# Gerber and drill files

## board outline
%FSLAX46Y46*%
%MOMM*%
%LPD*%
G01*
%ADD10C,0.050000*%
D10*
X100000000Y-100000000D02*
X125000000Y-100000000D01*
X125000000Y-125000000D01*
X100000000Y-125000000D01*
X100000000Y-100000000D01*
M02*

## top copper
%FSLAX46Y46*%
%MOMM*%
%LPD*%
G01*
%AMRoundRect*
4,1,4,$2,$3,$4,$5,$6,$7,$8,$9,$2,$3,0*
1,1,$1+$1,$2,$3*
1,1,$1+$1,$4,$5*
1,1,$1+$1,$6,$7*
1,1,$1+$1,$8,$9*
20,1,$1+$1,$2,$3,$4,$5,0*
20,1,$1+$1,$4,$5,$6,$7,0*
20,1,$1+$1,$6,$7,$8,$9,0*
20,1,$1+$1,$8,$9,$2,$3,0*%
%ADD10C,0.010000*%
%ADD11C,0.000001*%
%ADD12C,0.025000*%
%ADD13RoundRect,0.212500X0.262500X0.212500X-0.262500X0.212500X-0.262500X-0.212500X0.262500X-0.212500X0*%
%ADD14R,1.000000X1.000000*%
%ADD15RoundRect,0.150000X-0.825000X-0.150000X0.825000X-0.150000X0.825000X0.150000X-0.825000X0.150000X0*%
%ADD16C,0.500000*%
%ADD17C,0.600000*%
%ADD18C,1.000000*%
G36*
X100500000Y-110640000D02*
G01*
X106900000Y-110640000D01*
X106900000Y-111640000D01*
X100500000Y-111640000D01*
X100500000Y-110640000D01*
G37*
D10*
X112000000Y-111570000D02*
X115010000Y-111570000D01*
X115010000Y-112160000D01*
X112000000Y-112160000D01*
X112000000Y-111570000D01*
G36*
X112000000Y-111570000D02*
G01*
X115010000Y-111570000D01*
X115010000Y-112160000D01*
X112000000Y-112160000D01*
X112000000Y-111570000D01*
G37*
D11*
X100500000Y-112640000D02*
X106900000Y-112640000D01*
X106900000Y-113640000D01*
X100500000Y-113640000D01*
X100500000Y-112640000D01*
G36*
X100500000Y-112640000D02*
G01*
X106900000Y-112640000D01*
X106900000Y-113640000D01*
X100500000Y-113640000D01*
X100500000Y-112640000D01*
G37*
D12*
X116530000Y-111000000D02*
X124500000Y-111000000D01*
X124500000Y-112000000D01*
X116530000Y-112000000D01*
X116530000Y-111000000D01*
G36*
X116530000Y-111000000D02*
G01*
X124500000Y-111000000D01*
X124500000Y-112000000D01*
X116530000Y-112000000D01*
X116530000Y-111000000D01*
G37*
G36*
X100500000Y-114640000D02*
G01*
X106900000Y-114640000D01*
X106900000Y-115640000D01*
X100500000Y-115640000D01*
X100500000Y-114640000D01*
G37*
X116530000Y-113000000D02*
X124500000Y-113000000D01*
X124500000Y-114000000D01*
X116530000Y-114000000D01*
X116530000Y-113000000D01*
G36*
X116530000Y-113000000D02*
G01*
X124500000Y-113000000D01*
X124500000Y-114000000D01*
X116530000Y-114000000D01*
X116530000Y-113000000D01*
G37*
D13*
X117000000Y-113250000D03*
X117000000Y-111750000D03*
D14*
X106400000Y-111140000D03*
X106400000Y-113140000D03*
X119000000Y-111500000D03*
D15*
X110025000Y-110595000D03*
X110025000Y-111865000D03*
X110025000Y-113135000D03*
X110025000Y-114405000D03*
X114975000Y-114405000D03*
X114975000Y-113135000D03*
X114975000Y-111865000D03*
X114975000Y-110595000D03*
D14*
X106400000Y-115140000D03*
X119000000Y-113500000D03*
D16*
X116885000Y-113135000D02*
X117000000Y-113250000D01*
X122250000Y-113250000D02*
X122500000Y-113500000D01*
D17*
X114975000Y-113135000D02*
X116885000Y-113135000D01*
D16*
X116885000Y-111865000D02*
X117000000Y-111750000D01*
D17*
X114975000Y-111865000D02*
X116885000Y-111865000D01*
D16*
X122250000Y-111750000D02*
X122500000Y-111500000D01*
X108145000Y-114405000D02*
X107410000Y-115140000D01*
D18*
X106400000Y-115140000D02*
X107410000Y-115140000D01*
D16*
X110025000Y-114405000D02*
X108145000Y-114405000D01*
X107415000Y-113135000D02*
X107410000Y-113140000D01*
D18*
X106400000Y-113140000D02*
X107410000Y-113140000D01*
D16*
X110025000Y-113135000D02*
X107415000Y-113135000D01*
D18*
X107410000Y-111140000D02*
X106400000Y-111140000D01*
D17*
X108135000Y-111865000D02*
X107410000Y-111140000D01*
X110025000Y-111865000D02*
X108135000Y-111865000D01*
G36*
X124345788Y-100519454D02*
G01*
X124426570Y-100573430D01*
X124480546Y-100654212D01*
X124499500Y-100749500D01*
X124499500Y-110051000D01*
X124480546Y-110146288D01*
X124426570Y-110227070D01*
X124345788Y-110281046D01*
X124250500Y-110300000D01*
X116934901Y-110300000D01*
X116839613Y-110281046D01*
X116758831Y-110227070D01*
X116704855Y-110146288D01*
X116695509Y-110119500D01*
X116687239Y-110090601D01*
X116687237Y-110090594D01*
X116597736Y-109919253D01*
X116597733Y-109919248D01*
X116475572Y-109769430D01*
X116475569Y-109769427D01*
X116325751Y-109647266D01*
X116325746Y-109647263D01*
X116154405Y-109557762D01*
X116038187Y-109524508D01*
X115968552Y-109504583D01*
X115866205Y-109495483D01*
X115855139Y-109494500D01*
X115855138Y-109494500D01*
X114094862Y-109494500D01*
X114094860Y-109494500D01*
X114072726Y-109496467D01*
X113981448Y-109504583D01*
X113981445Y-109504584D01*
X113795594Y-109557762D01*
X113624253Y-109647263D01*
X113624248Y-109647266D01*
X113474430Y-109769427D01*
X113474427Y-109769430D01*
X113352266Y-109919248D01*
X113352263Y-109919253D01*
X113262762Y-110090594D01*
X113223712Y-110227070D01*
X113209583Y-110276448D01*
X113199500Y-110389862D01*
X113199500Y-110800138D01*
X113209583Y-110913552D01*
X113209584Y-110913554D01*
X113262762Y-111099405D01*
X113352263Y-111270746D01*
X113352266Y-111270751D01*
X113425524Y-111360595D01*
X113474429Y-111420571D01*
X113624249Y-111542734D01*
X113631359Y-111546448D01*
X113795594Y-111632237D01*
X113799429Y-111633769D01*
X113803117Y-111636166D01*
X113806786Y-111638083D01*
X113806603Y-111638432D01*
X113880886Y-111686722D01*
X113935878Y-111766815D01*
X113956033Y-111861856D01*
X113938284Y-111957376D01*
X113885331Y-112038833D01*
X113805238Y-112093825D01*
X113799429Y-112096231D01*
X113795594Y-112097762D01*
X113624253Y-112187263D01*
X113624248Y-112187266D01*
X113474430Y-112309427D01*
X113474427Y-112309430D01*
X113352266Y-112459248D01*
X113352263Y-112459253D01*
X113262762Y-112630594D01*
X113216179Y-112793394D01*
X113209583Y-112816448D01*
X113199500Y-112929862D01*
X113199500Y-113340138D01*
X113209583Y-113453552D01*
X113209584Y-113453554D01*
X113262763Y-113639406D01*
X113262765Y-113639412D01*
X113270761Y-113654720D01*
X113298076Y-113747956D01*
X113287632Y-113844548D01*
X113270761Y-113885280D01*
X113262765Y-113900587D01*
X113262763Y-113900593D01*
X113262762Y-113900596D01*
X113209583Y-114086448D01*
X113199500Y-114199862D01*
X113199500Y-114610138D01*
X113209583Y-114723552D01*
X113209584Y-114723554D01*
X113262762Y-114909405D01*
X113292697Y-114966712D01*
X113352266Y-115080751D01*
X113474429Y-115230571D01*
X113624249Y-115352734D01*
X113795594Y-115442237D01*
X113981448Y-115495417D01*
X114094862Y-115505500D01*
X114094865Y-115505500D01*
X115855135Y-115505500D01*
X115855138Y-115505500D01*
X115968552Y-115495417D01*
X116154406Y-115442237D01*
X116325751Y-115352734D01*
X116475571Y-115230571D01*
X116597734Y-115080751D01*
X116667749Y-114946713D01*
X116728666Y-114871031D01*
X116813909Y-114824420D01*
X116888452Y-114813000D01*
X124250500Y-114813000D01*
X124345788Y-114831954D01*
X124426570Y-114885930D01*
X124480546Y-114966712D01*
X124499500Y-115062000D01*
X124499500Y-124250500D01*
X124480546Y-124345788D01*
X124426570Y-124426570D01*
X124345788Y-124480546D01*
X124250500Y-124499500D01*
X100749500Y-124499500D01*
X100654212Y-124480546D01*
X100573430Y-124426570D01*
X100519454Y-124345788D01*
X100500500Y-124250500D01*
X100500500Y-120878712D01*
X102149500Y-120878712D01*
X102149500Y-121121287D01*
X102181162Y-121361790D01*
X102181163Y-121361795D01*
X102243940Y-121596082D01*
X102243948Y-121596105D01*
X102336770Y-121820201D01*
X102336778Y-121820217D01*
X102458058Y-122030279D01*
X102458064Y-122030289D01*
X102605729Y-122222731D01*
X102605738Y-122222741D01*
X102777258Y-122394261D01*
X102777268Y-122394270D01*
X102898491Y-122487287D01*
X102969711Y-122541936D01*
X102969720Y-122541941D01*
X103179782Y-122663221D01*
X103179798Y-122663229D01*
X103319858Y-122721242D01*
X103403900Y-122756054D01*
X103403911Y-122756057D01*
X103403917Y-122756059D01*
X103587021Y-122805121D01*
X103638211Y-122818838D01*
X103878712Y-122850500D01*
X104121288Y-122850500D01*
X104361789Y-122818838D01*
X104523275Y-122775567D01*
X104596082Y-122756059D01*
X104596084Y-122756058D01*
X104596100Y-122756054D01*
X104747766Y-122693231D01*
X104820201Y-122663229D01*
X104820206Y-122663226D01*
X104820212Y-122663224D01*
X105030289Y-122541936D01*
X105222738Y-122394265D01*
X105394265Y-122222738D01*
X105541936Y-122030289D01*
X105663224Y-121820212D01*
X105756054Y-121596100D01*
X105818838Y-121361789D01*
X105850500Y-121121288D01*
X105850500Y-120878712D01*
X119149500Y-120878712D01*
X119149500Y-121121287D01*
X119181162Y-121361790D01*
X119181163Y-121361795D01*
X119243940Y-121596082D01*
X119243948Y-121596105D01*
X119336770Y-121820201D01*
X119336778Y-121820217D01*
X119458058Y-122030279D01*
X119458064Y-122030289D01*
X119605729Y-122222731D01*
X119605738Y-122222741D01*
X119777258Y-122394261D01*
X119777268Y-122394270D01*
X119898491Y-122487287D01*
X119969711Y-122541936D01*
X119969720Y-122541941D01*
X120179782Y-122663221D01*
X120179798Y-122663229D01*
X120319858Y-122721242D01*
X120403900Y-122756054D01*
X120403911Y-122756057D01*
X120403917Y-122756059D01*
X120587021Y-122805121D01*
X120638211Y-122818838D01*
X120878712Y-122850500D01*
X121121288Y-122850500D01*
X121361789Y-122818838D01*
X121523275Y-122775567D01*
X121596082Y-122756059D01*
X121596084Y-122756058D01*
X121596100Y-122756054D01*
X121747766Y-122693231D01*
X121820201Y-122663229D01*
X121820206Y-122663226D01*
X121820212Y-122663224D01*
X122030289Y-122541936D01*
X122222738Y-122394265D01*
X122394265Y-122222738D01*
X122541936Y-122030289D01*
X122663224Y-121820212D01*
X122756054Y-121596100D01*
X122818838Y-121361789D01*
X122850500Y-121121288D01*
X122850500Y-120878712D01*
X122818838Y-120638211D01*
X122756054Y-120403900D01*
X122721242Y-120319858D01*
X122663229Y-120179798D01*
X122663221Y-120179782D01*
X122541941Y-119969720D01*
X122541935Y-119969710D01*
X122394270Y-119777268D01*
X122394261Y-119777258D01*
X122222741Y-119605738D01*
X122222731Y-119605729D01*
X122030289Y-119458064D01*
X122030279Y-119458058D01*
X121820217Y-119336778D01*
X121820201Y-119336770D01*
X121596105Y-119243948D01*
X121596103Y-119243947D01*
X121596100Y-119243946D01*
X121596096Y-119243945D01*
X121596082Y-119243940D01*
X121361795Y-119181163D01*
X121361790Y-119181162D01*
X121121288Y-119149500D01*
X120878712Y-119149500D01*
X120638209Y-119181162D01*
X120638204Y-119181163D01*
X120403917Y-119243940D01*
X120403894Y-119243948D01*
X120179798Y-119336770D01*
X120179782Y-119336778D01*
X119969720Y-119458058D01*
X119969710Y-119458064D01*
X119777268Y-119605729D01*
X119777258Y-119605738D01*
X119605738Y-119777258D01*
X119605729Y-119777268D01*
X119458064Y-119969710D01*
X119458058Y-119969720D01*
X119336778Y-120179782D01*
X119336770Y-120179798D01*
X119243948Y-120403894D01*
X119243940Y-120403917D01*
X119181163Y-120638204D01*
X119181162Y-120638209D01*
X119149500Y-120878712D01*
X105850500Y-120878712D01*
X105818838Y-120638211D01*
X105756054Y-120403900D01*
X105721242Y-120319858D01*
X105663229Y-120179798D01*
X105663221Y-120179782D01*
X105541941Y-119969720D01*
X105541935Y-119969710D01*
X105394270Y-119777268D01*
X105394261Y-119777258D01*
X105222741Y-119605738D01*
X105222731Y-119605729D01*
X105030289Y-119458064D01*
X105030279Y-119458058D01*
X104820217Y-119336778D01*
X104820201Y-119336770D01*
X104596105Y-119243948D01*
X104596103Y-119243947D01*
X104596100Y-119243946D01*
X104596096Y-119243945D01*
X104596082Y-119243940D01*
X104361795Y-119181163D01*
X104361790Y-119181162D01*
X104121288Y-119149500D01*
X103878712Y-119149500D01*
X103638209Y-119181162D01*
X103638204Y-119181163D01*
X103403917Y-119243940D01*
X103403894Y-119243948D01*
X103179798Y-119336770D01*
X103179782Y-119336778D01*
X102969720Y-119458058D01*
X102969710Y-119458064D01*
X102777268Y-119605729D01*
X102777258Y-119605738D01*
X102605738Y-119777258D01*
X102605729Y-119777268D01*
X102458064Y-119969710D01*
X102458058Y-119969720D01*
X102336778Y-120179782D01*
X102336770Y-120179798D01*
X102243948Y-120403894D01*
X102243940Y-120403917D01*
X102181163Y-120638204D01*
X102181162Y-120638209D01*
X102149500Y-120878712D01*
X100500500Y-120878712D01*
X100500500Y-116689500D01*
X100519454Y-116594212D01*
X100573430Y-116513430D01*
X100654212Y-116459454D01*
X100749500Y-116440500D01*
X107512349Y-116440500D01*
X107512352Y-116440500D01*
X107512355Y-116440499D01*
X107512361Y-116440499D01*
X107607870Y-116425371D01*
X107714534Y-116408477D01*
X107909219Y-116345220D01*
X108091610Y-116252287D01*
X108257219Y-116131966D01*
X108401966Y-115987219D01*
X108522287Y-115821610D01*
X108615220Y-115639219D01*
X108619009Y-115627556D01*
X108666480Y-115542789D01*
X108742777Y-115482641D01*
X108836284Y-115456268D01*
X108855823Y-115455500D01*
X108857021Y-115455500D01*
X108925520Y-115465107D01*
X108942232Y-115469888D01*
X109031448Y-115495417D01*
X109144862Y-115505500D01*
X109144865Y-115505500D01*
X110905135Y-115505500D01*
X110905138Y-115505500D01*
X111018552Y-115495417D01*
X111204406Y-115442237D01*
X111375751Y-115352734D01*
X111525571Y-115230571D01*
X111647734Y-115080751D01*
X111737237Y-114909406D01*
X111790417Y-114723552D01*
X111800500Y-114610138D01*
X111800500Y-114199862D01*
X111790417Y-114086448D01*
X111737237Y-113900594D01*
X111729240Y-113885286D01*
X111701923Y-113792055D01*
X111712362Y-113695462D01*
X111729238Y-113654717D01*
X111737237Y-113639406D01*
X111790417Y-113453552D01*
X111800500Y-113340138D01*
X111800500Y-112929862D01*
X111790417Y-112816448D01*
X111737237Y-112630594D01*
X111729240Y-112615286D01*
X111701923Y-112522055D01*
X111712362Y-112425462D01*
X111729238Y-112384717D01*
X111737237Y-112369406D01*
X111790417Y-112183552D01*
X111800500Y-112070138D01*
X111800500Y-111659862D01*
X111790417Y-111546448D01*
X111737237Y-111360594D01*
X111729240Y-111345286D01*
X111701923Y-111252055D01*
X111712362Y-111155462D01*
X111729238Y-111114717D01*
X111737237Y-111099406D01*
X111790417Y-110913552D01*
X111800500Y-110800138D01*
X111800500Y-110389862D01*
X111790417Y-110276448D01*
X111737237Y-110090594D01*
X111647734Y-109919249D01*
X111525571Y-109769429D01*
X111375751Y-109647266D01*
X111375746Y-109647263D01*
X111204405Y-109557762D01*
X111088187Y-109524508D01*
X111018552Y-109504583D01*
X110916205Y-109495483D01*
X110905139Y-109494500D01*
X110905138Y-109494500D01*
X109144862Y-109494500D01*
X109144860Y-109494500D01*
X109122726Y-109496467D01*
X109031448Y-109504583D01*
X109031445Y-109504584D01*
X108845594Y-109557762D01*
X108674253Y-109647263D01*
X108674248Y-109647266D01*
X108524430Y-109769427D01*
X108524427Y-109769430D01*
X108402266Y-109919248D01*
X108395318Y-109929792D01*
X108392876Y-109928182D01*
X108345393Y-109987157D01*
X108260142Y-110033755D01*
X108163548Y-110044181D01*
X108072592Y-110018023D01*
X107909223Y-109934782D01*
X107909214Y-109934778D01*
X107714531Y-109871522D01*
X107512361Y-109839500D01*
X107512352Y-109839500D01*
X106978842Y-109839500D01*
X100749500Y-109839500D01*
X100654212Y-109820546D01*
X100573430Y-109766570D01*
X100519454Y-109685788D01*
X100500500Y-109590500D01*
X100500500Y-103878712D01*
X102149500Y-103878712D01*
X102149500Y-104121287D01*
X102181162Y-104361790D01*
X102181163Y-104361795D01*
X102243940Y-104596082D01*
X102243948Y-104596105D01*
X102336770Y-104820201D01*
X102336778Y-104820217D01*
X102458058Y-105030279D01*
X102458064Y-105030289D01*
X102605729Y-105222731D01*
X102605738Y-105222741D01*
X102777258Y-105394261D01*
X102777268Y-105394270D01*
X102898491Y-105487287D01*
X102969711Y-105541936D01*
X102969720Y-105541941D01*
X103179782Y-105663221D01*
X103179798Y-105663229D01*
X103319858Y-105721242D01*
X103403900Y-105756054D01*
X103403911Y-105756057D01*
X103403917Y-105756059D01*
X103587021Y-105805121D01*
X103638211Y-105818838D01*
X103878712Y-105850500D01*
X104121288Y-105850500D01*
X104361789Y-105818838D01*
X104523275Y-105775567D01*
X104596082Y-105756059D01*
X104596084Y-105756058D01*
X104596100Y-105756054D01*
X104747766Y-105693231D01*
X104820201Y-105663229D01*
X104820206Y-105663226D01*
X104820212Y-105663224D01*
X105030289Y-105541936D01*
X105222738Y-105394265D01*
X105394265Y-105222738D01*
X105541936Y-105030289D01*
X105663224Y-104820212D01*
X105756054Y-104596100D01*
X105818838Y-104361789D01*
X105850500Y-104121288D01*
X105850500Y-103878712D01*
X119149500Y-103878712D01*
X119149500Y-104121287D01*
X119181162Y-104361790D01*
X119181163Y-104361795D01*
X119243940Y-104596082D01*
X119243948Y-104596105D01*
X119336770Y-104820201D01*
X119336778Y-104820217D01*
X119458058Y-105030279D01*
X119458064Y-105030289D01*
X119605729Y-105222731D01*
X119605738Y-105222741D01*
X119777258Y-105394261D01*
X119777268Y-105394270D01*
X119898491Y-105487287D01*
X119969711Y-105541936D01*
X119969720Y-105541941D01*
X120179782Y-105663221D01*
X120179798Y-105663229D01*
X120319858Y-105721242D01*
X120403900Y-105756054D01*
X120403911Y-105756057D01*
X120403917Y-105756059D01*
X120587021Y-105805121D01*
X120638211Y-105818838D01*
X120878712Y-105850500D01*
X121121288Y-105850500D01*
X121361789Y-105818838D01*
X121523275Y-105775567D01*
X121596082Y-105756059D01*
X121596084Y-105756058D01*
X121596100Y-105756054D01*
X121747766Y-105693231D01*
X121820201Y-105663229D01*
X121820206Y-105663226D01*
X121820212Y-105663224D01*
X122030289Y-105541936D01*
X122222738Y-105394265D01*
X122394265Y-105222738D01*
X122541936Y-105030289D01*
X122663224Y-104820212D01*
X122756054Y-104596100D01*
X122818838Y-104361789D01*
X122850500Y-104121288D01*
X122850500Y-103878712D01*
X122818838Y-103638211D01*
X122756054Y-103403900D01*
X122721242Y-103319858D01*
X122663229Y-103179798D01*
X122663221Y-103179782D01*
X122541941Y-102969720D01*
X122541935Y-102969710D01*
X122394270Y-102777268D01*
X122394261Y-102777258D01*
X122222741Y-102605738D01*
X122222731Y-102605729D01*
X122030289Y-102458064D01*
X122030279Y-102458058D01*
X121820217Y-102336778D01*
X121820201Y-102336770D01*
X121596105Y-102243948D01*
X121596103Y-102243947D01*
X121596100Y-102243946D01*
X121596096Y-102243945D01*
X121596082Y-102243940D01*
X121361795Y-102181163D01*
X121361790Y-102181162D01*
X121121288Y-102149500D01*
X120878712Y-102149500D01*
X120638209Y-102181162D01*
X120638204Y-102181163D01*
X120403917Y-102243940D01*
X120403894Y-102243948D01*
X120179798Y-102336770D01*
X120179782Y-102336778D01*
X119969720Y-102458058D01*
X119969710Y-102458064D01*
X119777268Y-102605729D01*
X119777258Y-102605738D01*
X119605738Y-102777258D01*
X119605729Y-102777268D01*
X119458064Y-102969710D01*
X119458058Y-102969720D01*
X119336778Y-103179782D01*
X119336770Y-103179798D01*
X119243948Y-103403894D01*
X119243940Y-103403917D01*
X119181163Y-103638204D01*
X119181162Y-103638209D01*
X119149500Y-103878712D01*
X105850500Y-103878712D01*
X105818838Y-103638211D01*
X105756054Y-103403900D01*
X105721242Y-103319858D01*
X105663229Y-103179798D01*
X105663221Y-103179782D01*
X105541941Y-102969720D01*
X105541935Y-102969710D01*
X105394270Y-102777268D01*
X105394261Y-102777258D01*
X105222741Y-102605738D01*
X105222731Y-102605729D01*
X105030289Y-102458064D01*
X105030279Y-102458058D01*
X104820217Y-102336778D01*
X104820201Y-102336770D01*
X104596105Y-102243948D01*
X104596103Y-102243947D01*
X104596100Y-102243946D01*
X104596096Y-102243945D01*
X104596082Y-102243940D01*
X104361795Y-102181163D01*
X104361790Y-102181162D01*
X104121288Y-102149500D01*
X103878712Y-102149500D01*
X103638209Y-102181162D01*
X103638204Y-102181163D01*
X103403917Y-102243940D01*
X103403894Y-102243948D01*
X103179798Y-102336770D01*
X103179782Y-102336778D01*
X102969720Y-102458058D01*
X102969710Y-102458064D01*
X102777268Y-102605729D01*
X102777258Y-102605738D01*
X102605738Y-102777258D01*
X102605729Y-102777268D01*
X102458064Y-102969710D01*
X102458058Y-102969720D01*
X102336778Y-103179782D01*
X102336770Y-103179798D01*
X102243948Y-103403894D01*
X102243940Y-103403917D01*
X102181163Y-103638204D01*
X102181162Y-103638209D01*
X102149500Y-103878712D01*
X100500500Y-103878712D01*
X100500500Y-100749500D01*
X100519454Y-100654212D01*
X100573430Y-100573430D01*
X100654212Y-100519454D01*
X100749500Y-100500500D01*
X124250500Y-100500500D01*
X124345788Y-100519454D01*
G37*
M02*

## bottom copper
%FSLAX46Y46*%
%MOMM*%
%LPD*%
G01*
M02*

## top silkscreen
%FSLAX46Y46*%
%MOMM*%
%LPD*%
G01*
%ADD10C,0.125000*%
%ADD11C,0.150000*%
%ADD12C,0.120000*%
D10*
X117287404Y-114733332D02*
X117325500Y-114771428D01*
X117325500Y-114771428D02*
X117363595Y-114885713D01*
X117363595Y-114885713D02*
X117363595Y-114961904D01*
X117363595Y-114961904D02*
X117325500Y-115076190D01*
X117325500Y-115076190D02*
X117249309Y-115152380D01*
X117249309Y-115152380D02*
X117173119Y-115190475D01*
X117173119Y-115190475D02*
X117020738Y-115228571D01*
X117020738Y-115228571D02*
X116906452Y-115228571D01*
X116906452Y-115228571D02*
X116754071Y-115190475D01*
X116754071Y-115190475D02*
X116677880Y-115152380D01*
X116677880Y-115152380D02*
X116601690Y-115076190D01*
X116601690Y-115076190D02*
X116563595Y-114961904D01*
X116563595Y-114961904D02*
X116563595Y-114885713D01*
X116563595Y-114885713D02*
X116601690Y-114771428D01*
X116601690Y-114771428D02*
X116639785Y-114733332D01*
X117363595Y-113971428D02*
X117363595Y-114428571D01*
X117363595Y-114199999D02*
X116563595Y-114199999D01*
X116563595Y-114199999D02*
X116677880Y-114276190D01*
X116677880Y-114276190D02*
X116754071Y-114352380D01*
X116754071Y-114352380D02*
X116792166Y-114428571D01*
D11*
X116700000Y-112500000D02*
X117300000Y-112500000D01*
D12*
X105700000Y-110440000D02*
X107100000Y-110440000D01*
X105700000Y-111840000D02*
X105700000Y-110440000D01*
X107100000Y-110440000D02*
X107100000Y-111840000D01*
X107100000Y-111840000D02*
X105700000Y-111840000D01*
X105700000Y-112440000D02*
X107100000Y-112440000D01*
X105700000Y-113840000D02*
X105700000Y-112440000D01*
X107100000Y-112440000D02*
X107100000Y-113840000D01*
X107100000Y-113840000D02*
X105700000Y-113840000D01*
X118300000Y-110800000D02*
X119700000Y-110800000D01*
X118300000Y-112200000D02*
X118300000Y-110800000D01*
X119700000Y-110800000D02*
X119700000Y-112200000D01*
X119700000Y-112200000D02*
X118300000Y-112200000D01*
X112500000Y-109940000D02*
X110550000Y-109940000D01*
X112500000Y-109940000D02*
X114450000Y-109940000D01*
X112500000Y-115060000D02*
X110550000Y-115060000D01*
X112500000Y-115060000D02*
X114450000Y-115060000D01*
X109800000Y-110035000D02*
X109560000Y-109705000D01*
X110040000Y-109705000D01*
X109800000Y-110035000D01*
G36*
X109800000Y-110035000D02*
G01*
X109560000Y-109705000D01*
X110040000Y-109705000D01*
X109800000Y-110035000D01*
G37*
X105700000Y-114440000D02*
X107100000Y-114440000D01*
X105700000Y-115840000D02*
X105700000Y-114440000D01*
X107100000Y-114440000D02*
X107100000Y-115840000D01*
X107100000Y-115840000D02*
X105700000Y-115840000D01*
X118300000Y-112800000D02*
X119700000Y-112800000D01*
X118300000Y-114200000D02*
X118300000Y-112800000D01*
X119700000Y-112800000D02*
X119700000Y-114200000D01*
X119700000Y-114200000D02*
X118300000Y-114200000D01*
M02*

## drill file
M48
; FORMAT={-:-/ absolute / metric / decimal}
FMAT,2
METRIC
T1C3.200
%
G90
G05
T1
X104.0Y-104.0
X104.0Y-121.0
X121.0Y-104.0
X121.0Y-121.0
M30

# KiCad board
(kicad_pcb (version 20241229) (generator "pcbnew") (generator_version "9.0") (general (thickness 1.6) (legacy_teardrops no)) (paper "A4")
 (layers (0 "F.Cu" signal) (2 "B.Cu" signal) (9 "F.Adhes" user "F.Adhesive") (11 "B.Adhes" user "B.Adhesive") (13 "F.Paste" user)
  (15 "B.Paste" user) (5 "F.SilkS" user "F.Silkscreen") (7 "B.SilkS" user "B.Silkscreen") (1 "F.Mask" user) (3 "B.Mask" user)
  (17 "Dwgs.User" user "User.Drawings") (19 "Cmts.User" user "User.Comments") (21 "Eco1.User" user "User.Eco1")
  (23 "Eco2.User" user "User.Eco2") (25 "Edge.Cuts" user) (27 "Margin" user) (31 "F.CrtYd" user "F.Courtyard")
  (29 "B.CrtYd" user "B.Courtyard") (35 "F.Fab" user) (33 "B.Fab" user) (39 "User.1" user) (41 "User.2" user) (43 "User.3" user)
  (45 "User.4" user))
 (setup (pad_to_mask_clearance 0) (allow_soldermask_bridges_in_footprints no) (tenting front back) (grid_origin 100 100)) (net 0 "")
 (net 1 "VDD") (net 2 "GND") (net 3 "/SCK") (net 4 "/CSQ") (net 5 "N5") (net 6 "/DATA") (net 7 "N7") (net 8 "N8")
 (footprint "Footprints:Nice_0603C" (layer "F.Cu") (at 117 112.5 90)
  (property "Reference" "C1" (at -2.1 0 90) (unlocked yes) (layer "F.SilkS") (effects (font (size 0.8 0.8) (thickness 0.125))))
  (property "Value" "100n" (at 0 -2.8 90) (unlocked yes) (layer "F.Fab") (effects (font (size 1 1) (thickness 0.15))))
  (fp_line (start 0 -0.3) (end 0 0.3) (stroke (width 0.15) (type default)) (layer "F.SilkS"))
  (pad "1" smd roundrect (at -0.75 0 180) (size 0.95 0.85) (layers "F.Cu" "F.Mask" "F.Paste") (roundrect_rratio 0.25) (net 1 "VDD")
   (thermal_bridge_angle 45))
  (pad "2" smd roundrect (at 0.75 0 180) (size 0.95 0.85) (layers "F.Cu" "F.Mask" "F.Paste") (roundrect_rratio 0.25) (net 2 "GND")
   (thermal_bridge_angle 45)))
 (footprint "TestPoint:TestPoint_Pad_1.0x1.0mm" (layer "F.Cu") (at 106.4 111.14)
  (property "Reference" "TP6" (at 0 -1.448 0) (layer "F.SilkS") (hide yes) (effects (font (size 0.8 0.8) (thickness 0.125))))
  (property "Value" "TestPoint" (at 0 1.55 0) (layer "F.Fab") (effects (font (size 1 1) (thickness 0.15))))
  (fp_line (start -0.7 -0.7) (end 0.7 -0.7) (stroke (width 0.12) (type solid)) (layer "F.SilkS"))
  (fp_line (start -0.7 0.7) (end -0.7 -0.7) (stroke (width 0.12) (type solid)) (layer "F.SilkS"))
  (fp_line (start 0.7 -0.7) (end 0.7 0.7) (stroke (width 0.12) (type solid)) (layer "F.SilkS"))
  (fp_line (start 0.7 0.7) (end -0.7 0.7) (stroke (width 0.12) (type solid)) (layer "F.SilkS"))
  (pad "1" smd rect (at 0 0) (size 1 1) (layers "F.Cu" "F.Mask") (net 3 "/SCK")))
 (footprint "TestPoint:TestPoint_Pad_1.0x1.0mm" (layer "F.Cu") (at 106.4 113.14)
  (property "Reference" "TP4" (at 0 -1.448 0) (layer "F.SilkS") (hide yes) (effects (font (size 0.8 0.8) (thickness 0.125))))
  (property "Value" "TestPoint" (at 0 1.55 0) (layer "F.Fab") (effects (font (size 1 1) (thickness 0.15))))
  (fp_line (start -0.7 -0.7) (end 0.7 -0.7) (stroke (width 0.12) (type solid)) (layer "F.SilkS"))
  (fp_line (start -0.7 0.7) (end -0.7 -0.7) (stroke (width 0.12) (type solid)) (layer "F.SilkS"))
  (fp_line (start 0.7 -0.7) (end 0.7 0.7) (stroke (width 0.12) (type solid)) (layer "F.SilkS"))
  (fp_line (start 0.7 0.7) (end -0.7 0.7) (stroke (width 0.12) (type solid)) (layer "F.SilkS"))
  (pad "1" smd rect (at 0 0) (size 1 1) (layers "F.Cu" "F.Mask") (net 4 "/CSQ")))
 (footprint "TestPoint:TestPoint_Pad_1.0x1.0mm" (layer "F.Cu") (at 119 111.5)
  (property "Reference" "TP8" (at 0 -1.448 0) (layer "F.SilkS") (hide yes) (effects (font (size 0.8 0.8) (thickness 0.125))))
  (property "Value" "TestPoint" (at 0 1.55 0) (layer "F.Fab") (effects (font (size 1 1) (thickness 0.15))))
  (fp_line (start -0.7 -0.7) (end 0.7 -0.7) (stroke (width 0.12) (type solid)) (layer "F.SilkS"))
  (fp_line (start -0.7 0.7) (end -0.7 -0.7) (stroke (width 0.12) (type solid)) (layer "F.SilkS"))
  (fp_line (start 0.7 -0.7) (end 0.7 0.7) (stroke (width 0.12) (type solid)) (layer "F.SilkS"))
  (fp_line (start 0.7 0.7) (end -0.7 0.7) (stroke (width 0.12) (type solid)) (layer "F.SilkS"))
  (pad "1" smd rect (at 0 0) (size 1 1) (layers "F.Cu" "F.Mask") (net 2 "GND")))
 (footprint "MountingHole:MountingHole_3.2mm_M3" (layer "F.Cu") (at 104 104)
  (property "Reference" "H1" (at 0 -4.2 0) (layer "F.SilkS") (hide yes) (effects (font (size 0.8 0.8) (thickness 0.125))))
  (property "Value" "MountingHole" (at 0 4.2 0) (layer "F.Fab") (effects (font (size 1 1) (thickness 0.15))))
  (pad "" np_thru_hole circle (at 0 0) (size 3.2 3.2) (drill 3.2) (layers "*.Cu" "*.Mask")))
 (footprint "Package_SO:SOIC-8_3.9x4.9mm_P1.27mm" (layer "F.Cu") (at 112.5 112.5)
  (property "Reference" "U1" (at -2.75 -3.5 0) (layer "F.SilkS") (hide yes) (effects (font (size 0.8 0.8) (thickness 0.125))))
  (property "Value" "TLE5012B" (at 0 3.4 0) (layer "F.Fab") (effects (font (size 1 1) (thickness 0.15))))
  (fp_line (start 0 -2.56) (end -1.95 -2.56) (stroke (width 0.12) (type solid)) (layer "F.SilkS"))
  (fp_line (start 0 -2.56) (end 1.95 -2.56) (stroke (width 0.12) (type solid)) (layer "F.SilkS"))
  (fp_line (start 0 2.56) (end -1.95 2.56) (stroke (width 0.12) (type solid)) (layer "F.SilkS"))
  (fp_line (start 0 2.56) (end 1.95 2.56) (stroke (width 0.12) (type solid)) (layer "F.SilkS"))
  (fp_poly
   (pts (xy -2.7 -2.465) (xy -2.94 -2.795) (xy -2.46 -2.795) (xy -2.7 -2.465)) (stroke (width 0.12) (type solid)) (fill yes)
   (layer "F.SilkS"))
  (pad "1" smd roundrect (at -2.475 -1.905) (size 1.95 0.6) (layers "F.Cu" "F.Mask" "F.Paste") (roundrect_rratio 0.25) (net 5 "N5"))
  (pad "2" smd roundrect (at -2.475 -0.635) (size 1.95 0.6) (layers "F.Cu" "F.Mask" "F.Paste") (roundrect_rratio 0.25) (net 3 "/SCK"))
  (pad "3" smd roundrect (at -2.475 0.635) (size 1.95 0.6) (layers "F.Cu" "F.Mask" "F.Paste") (roundrect_rratio 0.25) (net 4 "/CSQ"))
  (pad "4" smd roundrect (at -2.475 1.905) (size 1.95 0.6) (layers "F.Cu" "F.Mask" "F.Paste") (roundrect_rratio 0.25) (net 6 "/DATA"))
  (pad "5" smd roundrect (at 2.475 1.905) (size 1.95 0.6) (layers "F.Cu" "F.Mask" "F.Paste") (roundrect_rratio 0.25) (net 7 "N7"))
  (pad "6" smd roundrect (at 2.475 0.635) (size 1.95 0.6) (layers "F.Cu" "F.Mask" "F.Paste") (roundrect_rratio 0.25) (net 1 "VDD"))
  (pad "7" smd roundrect (at 2.475 -0.635) (size 1.95 0.6) (layers "F.Cu" "F.Mask" "F.Paste") (roundrect_rratio 0.25) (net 2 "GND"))
  (pad "8" smd roundrect (at 2.475 -1.905) (size 1.95 0.6) (layers "F.Cu" "F.Mask" "F.Paste") (roundrect_rratio 0.25) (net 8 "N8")))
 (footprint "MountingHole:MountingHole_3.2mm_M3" (layer "F.Cu") (at 121 104)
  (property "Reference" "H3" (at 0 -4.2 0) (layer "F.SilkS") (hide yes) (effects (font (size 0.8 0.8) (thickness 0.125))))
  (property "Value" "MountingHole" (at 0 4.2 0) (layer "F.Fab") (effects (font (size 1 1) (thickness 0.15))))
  (pad "" np_thru_hole circle (at 0 0) (size 3.2 3.2) (drill 3.2) (layers "*.Cu" "*.Mask")))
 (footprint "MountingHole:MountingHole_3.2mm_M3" (layer "F.Cu") (at 121 121)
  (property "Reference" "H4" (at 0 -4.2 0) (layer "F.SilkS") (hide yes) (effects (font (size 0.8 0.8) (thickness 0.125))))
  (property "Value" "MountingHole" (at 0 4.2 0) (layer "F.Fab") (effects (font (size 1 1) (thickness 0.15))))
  (pad "" np_thru_hole circle (at 0 0) (size 3.2 3.2) (drill 3.2) (layers "*.Cu" "*.Mask")))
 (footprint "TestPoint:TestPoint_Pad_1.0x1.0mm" (layer "F.Cu") (at 106.4 115.14)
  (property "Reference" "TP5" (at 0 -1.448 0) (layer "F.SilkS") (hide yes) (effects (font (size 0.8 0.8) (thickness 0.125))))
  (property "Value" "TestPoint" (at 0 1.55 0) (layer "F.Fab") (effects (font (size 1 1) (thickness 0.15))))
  (fp_line (start -0.7 -0.7) (end 0.7 -0.7) (stroke (width 0.12) (type solid)) (layer "F.SilkS"))
  (fp_line (start -0.7 0.7) (end -0.7 -0.7) (stroke (width 0.12) (type solid)) (layer "F.SilkS"))
  (fp_line (start 0.7 -0.7) (end 0.7 0.7) (stroke (width 0.12) (type solid)) (layer "F.SilkS"))
  (fp_line (start 0.7 0.7) (end -0.7 0.7) (stroke (width 0.12) (type solid)) (layer "F.SilkS"))
  (pad "1" smd rect (at 0 0) (size 1 1) (layers "F.Cu" "F.Mask") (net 6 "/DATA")))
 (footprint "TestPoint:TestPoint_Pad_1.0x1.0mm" (layer "F.Cu") (at 119 113.5)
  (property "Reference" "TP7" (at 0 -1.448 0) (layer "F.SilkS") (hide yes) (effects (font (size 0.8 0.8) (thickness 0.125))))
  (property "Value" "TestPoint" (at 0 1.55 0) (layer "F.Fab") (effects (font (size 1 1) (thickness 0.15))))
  (fp_line (start -0.7 -0.7) (end 0.7 -0.7) (stroke (width 0.12) (type solid)) (layer "F.SilkS"))
  (fp_line (start -0.7 0.7) (end -0.7 -0.7) (stroke (width 0.12) (type solid)) (layer "F.SilkS"))
  (fp_line (start 0.7 -0.7) (end 0.7 0.7) (stroke (width 0.12) (type solid)) (layer "F.SilkS"))
  (fp_line (start 0.7 0.7) (end -0.7 0.7) (stroke (width 0.12) (type solid)) (layer "F.SilkS"))
  (pad "1" smd rect (at 0 0) (size 1 1) (layers "F.Cu" "F.Mask") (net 1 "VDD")))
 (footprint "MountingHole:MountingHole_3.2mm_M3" (layer "F.Cu") (at 104 121)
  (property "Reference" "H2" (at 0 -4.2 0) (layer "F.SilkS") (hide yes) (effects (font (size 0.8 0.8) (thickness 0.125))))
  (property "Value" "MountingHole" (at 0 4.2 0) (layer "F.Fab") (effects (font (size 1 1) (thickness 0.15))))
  (pad "" np_thru_hole circle (at 0 0) (size 3.2 3.2) (drill 3.2) (layers "*.Cu" "*.Mask")))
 (gr_rect (start 100.5 110.64) (end 106.9 111.64) (stroke (width 0) (type solid)) (fill yes) (layer "F.Cu") (net 3))
 (gr_rect (start 112 111.57) (end 115.01 112.16) (stroke (width 0.01) (type solid)) (fill yes) (layer "F.Cu") (net 2))
 (gr_rect (start 100.5 112.64) (end 106.9 113.64) (stroke (width 0.000001) (type solid)) (fill yes) (layer "F.Cu") (net 4))
 (gr_rect (start 116.53 111) (end 124.5 112) (stroke (width 0.025) (type solid)) (fill yes) (layer "F.Cu") (net 2))
 (gr_rect (start 100.5 114.64) (end 106.9 115.64) (stroke (width 0) (type solid)) (fill yes) (layer "F.Cu") (net 6))
 (gr_rect (start 116.53 113) (end 124.5 114) (stroke (width 0.025) (type solid)) (fill yes) (layer "F.Cu") (net 1))
 (gr_rect (start 100 100) (end 125 125) (stroke (width 0.05) (type solid)) (fill no) (layer "Edge.Cuts"))
 (segment (start 116.885 113.135) (end 117 113.25) (width 0.5) (layer "F.Cu") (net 1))
 (segment (start 122.25 113.25) (end 122.5 113.5) (width 0.5) (layer "F.Cu") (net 1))
 (segment (start 114.975 113.135) (end 116.885 113.135) (width 0.6) (layer "F.Cu") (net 1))
 (segment (start 116.885 111.865) (end 117 111.75) (width 0.5) (layer "F.Cu") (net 2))
 (segment (start 114.975 111.865) (end 116.885 111.865) (width 0.6) (layer "F.Cu") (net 2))
 (segment (start 122.25 111.75) (end 122.5 111.5) (width 0.5) (layer "F.Cu") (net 2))
 (segment (start 108.145 114.405) (end 107.41 115.14) (width 0.5) (layer "F.Cu") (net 6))
 (segment (start 106.4 115.14) (end 107.41 115.14) (width 1) (layer "F.Cu") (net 6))
 (segment (start 110.025 114.405) (end 108.145 114.405) (width 0.5) (layer "F.Cu") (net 6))
 (segment (start 107.415 113.135) (end 107.41 113.14) (width 0.5) (layer "F.Cu") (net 4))
 (segment (start 106.4 113.14) (end 107.41 113.14) (width 1) (layer "F.Cu") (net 4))
 (segment (start 110.025 113.135) (end 107.415 113.135) (width 0.5) (layer "F.Cu") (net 4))
 (segment (start 107.41 111.14) (end 106.4 111.14) (width 1) (layer "F.Cu") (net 3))
 (segment (start 108.135 111.865) (end 107.41 111.14) (width 0.6) (layer "F.Cu") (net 3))
 (segment (start 110.025 111.865) (end 108.135 111.865) (width 0.6) (layer "F.Cu") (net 3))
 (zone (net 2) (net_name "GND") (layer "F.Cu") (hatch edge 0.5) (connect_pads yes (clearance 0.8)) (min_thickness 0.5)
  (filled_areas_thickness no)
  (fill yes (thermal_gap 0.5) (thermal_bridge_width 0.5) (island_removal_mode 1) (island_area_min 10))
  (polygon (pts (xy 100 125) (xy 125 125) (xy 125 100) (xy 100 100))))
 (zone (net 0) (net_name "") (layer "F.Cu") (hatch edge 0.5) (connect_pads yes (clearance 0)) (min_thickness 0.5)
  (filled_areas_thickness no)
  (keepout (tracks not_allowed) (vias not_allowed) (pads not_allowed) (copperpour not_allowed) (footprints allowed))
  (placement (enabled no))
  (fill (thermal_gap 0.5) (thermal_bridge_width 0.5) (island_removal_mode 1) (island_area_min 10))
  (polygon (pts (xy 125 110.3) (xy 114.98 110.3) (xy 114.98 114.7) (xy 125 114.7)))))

